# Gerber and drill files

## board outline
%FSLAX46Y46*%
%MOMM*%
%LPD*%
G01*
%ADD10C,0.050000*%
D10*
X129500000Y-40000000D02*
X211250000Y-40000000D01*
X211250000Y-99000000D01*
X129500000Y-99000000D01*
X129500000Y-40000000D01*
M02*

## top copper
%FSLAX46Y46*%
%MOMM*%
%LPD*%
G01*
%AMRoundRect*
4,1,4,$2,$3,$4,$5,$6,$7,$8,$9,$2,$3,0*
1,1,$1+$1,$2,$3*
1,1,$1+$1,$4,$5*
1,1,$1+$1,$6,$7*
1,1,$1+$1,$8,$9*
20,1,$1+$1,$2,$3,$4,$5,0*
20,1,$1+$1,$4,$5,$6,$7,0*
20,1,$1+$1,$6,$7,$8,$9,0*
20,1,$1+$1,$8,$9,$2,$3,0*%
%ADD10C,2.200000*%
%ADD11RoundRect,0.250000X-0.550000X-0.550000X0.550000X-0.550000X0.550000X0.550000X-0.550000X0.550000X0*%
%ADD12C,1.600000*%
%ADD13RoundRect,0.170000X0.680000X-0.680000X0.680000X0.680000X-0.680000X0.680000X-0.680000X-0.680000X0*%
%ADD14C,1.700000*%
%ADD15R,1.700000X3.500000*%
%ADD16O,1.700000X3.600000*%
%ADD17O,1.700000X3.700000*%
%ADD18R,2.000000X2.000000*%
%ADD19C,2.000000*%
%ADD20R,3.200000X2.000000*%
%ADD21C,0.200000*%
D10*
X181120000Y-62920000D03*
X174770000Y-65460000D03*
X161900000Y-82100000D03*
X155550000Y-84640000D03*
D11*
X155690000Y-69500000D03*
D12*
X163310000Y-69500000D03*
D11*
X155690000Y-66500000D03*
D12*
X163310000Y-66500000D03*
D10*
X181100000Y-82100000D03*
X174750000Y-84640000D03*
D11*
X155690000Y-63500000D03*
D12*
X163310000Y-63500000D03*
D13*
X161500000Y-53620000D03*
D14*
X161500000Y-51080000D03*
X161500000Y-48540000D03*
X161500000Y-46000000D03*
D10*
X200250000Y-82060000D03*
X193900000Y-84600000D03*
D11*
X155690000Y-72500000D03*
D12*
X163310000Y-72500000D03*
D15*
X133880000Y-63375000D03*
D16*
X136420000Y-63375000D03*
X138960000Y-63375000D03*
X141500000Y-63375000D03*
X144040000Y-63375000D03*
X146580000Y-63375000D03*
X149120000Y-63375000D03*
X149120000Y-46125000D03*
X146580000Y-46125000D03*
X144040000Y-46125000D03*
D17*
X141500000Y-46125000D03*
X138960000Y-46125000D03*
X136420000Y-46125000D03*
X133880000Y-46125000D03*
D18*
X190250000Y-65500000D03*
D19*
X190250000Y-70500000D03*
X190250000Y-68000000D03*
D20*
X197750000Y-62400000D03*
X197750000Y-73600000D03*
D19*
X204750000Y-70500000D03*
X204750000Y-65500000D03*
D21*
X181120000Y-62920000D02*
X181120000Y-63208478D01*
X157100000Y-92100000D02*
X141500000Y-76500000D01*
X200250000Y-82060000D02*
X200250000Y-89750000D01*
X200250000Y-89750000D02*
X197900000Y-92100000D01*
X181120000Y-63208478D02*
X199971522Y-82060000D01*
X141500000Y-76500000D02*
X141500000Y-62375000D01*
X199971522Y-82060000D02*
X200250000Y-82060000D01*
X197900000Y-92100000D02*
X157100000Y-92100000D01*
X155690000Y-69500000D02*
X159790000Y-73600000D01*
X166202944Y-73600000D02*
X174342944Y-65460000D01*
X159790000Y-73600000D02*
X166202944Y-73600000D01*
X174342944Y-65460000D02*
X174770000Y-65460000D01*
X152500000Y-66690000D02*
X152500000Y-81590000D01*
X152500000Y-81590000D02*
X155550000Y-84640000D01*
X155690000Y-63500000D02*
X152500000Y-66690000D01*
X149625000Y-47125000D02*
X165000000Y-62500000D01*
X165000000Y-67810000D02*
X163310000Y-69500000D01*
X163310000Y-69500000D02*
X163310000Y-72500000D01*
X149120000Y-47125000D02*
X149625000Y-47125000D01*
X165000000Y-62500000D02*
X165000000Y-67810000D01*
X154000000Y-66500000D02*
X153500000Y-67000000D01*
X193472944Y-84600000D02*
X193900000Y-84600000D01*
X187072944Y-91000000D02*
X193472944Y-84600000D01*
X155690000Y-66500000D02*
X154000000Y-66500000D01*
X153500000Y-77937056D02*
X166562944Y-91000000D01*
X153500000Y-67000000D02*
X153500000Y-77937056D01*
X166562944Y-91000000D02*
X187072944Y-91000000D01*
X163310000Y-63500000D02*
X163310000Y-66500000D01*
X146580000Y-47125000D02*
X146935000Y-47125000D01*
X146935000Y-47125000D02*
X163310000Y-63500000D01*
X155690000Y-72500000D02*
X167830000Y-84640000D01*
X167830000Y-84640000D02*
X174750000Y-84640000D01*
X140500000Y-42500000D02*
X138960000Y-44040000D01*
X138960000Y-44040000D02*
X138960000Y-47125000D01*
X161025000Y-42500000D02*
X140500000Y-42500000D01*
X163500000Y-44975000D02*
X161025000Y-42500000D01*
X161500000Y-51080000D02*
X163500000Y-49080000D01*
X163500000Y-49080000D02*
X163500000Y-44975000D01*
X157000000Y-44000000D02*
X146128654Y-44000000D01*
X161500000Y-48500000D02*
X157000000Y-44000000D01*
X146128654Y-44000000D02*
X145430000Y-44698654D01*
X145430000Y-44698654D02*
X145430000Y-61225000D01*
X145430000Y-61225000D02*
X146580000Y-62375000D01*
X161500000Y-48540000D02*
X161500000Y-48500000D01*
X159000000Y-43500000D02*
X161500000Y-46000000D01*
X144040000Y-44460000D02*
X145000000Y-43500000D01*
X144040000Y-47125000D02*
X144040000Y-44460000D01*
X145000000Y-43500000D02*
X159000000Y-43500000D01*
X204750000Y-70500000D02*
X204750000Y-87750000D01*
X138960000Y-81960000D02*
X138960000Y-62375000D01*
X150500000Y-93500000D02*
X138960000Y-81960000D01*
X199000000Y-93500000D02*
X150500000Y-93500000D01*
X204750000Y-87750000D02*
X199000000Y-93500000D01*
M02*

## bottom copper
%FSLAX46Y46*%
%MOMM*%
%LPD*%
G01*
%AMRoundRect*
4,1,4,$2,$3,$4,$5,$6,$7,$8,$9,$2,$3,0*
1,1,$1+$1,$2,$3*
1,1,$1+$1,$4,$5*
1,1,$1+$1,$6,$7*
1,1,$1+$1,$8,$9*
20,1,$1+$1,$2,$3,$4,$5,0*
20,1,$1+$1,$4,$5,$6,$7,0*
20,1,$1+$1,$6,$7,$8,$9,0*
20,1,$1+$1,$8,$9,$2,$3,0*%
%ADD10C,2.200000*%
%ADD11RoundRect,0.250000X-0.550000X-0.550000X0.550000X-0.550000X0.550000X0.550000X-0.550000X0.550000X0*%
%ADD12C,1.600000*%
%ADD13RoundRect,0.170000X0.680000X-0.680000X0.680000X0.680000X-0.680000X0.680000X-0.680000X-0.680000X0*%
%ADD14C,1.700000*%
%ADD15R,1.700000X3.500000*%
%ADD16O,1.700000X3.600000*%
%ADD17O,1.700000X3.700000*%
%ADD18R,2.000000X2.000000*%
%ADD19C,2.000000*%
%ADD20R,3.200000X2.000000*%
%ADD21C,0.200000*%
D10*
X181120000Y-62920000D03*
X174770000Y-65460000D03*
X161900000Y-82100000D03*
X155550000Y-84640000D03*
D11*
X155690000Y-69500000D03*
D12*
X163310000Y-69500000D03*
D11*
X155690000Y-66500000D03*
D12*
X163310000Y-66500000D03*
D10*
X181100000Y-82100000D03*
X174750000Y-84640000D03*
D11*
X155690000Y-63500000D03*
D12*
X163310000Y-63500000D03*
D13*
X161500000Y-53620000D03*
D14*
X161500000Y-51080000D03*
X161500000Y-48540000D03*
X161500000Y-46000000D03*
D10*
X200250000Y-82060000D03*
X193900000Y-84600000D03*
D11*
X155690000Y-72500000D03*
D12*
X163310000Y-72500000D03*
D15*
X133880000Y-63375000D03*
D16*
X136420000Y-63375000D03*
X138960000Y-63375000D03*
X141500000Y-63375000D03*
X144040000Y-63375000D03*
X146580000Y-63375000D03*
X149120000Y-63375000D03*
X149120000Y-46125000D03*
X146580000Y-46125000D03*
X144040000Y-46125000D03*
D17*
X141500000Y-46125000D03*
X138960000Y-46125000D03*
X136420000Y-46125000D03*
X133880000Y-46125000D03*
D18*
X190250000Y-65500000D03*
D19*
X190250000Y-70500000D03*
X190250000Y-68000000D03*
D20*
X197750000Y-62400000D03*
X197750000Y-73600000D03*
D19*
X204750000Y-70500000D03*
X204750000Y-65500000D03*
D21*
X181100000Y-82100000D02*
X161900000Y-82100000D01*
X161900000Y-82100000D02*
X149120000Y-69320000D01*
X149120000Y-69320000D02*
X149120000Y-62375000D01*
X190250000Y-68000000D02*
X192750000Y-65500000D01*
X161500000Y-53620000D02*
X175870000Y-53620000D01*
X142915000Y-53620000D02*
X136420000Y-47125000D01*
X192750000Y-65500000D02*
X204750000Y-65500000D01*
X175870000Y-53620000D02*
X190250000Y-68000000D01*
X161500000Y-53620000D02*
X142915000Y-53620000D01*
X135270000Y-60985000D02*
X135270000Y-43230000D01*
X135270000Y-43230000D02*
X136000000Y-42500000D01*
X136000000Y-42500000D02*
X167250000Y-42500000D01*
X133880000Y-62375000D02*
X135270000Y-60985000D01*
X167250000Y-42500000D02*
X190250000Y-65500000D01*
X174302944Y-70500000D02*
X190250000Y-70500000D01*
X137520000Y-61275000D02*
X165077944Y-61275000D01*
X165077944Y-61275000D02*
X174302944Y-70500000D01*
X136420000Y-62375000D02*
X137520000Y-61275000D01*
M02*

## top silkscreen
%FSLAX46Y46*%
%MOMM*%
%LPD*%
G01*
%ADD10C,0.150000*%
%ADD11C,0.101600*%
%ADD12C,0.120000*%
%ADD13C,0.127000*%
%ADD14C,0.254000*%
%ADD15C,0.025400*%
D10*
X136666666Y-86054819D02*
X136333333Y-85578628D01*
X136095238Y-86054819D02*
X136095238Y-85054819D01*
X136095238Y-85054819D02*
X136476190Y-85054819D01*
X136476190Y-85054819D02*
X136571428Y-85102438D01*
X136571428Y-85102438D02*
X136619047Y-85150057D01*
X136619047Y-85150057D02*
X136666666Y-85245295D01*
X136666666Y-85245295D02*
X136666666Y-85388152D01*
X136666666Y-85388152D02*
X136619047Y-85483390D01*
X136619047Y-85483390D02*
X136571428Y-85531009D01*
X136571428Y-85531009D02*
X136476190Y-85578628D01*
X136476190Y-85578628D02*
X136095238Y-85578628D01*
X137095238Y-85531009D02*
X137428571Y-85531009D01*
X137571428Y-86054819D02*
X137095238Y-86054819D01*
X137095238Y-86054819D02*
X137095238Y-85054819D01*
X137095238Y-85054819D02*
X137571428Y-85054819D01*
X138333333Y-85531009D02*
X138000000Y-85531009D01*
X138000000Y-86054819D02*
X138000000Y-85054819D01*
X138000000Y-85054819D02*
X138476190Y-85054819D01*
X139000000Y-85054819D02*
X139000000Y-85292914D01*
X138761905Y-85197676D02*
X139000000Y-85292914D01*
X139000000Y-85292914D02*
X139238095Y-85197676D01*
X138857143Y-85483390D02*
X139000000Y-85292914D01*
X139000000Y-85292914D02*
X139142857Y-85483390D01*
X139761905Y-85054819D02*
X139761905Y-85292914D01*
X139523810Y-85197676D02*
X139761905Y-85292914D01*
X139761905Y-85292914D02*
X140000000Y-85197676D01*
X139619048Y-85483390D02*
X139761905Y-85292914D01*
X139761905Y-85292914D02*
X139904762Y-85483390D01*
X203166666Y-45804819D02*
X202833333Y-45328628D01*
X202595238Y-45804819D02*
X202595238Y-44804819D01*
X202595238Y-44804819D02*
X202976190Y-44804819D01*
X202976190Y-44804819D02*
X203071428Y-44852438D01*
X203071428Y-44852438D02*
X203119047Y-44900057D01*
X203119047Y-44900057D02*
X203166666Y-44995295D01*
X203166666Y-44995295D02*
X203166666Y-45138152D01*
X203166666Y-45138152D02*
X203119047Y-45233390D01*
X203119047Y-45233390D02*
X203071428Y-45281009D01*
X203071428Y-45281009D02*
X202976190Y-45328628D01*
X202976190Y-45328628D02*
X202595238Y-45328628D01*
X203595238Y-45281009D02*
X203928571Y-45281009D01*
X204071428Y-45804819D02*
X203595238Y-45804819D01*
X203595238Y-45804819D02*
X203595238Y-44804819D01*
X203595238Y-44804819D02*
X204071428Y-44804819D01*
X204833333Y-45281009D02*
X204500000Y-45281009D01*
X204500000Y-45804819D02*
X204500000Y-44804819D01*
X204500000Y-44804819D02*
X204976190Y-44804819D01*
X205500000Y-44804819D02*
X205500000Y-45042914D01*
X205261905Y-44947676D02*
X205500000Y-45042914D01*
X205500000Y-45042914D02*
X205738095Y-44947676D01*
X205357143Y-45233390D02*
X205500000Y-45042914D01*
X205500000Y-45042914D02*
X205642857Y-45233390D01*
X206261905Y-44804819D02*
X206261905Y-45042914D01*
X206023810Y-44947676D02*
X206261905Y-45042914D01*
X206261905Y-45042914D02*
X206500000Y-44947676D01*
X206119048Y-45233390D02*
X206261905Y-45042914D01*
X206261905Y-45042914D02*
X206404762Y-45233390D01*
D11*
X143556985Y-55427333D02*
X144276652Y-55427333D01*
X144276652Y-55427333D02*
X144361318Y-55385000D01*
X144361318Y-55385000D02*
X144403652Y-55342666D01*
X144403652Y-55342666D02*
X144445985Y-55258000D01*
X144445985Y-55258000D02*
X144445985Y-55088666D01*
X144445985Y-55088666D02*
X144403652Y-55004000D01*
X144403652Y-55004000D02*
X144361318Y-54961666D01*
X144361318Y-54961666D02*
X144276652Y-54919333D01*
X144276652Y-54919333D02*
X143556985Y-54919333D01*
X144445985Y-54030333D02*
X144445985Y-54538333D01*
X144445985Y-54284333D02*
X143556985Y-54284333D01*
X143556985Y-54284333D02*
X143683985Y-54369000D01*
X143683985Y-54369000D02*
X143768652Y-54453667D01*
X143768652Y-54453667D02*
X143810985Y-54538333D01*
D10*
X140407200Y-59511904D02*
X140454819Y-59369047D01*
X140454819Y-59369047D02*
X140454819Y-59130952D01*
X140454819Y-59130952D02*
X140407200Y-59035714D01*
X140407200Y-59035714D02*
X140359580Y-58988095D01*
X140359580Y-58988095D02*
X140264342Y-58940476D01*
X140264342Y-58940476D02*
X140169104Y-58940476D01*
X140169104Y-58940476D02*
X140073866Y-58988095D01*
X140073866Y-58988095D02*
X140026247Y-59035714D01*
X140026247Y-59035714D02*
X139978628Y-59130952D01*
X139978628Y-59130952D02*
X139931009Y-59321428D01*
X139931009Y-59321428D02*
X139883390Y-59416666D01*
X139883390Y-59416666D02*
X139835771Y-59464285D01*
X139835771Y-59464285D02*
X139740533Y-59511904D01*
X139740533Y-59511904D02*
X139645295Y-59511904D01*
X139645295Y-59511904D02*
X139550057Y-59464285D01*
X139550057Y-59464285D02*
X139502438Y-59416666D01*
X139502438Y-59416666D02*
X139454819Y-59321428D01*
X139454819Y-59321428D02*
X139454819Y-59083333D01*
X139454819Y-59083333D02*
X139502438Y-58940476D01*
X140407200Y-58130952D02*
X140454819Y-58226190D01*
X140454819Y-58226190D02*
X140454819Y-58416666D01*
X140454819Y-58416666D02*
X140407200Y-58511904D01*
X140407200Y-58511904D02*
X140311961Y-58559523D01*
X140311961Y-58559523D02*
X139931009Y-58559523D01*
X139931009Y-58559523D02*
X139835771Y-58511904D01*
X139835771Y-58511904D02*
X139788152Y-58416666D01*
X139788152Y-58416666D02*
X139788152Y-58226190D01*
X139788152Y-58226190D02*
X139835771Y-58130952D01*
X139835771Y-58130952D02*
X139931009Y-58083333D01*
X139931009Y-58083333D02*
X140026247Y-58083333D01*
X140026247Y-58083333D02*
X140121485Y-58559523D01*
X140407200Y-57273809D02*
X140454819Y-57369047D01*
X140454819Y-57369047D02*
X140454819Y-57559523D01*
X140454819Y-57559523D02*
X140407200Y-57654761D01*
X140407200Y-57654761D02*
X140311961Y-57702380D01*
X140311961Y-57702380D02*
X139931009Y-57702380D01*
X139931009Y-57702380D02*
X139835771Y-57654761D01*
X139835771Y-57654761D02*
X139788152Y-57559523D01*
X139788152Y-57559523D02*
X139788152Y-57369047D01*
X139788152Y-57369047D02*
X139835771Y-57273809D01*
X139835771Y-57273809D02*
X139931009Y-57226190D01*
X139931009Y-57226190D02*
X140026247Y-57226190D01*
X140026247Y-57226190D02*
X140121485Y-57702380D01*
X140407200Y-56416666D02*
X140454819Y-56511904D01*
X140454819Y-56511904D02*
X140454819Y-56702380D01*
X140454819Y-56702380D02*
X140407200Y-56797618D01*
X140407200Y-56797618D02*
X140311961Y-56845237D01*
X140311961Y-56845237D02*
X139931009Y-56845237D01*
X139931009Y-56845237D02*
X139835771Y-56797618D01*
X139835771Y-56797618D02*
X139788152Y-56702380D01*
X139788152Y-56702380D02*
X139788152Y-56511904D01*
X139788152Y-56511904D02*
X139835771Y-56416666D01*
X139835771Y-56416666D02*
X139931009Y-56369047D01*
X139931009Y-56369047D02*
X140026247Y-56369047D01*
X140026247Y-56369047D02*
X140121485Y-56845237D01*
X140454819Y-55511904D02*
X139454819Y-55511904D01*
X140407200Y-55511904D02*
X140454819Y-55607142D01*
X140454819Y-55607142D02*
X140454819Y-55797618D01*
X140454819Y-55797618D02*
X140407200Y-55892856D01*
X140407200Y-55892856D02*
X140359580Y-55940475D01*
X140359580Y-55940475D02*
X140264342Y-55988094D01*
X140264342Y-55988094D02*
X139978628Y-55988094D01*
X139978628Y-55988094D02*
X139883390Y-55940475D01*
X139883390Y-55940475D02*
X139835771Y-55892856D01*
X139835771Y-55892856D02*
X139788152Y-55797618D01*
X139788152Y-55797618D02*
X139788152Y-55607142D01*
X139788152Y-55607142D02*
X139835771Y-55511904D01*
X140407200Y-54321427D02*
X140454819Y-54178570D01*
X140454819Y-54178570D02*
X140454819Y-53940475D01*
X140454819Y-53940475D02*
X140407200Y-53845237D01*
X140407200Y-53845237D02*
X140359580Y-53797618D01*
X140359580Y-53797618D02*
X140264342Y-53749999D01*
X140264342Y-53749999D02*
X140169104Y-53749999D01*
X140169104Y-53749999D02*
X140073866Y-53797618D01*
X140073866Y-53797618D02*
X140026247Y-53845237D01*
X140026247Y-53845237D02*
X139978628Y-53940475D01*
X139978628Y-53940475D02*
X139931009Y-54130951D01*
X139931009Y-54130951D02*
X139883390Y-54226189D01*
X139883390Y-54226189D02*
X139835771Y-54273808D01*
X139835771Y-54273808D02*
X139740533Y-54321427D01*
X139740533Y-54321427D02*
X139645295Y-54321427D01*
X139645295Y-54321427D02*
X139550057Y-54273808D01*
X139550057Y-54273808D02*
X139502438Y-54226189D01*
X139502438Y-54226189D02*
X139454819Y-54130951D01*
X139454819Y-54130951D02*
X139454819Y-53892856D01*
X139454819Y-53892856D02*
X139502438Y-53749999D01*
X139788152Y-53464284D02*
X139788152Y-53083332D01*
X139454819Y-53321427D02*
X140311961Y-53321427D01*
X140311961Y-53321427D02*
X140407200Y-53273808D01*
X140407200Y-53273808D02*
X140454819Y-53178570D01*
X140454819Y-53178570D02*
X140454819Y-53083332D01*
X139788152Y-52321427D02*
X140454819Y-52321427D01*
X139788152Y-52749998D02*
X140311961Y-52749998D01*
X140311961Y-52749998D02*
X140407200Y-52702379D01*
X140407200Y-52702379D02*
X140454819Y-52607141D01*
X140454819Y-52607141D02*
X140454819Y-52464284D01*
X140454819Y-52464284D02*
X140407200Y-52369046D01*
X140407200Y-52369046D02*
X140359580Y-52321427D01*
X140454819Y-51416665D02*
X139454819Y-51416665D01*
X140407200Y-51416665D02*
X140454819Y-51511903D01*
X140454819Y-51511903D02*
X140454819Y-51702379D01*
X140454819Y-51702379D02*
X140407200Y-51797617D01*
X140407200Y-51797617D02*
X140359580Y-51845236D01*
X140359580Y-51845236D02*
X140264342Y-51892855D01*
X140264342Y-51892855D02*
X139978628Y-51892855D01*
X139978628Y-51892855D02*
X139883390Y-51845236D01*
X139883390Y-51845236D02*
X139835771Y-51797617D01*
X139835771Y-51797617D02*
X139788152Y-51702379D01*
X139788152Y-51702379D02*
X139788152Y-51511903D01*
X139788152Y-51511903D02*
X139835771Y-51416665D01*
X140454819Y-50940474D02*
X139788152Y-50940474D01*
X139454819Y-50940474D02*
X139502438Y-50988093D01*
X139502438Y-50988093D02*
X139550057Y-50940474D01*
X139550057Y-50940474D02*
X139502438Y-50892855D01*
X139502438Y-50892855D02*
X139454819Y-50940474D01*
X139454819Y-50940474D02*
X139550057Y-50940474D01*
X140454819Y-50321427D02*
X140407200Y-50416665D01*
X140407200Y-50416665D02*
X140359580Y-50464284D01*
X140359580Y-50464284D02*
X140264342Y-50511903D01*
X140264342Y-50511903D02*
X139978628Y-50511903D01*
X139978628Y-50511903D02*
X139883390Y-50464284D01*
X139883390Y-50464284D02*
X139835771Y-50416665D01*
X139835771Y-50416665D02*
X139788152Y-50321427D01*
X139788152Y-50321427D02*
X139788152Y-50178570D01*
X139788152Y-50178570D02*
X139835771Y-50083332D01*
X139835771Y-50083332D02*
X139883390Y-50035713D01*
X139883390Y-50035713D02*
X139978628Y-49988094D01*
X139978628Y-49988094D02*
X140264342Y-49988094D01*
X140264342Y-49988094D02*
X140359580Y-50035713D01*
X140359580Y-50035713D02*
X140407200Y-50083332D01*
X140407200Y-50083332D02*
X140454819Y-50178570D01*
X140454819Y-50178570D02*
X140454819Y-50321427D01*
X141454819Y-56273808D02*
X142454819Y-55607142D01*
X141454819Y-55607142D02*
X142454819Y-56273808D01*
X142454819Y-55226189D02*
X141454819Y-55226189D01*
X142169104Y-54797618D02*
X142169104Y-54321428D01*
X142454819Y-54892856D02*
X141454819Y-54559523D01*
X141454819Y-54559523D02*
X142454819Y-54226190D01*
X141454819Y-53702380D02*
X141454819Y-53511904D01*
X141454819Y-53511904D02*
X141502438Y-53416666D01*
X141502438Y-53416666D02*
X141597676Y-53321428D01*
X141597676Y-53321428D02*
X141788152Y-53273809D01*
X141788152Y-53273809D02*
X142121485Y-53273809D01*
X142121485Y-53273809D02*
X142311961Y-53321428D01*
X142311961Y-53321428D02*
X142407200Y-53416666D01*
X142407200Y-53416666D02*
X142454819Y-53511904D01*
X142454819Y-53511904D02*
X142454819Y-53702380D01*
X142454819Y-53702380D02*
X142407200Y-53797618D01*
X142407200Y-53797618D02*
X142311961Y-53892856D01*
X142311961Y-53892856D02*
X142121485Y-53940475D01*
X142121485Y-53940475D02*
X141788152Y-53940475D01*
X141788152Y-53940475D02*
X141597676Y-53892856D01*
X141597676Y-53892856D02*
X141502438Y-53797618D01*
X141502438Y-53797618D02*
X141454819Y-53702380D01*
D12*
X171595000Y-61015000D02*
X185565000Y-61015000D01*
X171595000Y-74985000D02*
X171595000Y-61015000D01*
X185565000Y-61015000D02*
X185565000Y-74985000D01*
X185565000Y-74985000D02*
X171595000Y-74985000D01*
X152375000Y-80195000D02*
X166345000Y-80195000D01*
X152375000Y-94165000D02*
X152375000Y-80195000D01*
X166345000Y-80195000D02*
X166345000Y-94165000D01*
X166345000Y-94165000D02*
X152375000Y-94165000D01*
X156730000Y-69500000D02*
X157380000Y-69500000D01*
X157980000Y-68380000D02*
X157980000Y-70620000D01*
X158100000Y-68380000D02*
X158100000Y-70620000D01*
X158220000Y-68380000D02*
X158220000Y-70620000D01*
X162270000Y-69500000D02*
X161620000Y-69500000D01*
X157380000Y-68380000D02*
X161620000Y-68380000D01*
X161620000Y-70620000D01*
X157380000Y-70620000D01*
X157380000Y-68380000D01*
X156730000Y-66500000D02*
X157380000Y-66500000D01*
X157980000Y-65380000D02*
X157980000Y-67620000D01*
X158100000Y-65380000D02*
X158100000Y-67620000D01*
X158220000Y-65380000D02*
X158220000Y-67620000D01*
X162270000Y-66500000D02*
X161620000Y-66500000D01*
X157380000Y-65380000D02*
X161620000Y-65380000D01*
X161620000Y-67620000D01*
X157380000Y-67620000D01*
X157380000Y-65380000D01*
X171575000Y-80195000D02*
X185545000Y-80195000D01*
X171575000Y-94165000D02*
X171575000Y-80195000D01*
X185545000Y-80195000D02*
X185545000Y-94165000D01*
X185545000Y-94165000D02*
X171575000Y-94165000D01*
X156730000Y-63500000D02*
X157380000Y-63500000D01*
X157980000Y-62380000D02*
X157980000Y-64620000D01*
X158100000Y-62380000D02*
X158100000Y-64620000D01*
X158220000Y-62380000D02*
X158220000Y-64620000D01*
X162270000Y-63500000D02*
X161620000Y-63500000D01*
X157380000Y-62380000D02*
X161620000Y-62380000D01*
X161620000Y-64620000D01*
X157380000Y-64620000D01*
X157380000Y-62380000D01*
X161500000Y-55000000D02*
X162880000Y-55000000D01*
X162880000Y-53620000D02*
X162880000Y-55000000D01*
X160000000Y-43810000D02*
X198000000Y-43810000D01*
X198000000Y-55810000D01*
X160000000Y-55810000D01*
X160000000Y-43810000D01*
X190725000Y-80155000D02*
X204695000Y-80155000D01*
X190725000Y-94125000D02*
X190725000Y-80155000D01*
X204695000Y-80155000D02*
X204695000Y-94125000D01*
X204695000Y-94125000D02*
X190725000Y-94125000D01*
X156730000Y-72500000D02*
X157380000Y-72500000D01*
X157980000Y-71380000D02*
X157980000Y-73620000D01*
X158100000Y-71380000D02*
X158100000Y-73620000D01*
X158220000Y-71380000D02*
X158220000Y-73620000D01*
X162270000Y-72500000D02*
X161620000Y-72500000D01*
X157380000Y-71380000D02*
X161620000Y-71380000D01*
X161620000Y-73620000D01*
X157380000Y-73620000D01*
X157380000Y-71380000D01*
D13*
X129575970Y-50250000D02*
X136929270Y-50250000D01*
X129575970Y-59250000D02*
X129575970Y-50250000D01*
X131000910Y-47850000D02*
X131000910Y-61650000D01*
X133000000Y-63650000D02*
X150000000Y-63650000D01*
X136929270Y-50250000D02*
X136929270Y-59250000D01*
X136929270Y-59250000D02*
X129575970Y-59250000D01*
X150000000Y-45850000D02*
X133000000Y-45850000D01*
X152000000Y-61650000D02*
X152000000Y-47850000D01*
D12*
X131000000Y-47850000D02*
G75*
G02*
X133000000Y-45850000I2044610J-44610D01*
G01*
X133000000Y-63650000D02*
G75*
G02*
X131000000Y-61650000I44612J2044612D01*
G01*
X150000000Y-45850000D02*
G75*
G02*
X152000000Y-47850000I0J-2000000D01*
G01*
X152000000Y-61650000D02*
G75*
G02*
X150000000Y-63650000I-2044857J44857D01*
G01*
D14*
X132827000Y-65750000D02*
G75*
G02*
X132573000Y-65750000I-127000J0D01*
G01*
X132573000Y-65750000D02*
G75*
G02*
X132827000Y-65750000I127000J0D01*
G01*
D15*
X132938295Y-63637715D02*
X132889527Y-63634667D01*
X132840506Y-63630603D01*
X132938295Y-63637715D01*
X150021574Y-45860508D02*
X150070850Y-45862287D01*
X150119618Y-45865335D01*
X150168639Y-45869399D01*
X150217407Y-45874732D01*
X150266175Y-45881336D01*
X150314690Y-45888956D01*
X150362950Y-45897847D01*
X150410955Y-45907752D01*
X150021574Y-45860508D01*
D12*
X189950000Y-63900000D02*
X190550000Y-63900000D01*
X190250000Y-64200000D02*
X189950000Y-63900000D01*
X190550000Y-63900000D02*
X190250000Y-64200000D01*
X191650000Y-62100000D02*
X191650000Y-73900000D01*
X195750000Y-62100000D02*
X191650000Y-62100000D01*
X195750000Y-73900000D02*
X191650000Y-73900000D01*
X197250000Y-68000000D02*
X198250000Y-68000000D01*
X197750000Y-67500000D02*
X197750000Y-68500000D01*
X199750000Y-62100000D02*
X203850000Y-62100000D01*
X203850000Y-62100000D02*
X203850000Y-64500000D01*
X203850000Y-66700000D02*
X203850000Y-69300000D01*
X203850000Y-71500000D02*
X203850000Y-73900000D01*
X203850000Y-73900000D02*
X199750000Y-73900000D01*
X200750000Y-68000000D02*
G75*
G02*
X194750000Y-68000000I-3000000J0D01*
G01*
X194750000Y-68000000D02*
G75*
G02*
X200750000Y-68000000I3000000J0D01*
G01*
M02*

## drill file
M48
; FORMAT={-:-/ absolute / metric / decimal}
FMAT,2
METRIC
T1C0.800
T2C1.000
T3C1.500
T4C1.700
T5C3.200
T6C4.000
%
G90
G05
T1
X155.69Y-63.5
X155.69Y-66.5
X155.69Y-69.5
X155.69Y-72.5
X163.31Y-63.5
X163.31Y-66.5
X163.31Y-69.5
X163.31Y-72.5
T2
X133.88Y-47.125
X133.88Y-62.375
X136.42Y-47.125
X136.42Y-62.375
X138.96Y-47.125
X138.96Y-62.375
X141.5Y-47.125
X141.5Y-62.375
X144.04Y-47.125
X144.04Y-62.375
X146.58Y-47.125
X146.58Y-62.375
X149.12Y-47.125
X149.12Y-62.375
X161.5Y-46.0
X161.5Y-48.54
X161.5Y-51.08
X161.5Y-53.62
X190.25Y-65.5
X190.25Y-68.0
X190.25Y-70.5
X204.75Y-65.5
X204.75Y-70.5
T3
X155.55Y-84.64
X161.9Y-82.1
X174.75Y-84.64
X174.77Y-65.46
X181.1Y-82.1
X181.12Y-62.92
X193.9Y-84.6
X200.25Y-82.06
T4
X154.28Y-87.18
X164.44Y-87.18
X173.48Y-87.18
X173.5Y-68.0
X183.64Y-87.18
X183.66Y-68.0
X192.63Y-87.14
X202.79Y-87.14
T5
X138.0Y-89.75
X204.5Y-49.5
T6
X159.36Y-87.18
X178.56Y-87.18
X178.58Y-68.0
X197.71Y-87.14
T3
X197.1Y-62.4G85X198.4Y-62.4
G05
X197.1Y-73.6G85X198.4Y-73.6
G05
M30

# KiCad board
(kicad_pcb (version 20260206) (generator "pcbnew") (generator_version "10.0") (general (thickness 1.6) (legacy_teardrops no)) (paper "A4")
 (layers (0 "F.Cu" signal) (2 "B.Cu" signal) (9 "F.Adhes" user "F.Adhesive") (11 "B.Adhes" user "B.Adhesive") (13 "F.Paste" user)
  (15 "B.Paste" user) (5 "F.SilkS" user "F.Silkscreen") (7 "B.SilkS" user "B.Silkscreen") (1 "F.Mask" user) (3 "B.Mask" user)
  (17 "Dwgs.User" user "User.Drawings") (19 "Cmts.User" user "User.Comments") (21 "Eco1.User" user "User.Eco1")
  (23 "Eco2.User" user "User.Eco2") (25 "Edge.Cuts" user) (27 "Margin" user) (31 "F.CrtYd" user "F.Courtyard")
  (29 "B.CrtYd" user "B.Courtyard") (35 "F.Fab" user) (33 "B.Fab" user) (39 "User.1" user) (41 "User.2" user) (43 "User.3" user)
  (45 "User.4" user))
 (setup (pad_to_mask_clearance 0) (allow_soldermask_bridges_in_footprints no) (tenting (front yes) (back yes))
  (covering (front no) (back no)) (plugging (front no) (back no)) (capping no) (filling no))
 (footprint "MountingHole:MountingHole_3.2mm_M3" (layer "F.Cu") (at 138 89.75)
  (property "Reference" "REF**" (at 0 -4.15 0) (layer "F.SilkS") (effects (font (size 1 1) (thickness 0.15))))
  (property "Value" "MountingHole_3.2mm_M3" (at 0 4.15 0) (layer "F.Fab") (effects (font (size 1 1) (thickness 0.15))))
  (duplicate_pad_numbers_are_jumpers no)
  (pad "" np_thru_hole circle (at 0 0) (size 3.2 3.2) (drill 3.2) (layers "*.Cu" "*.Mask")))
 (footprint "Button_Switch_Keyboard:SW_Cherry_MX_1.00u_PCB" (layer "F.Cu") (at 181.12 62.92)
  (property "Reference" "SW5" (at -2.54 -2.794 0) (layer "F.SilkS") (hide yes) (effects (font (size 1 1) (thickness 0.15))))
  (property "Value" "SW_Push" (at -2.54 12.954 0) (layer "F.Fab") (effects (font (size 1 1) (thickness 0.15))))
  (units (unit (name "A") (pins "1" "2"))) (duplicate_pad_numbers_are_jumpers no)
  (fp_line (start -9.525 -1.905) (end 4.445 -1.905) (stroke (width 0.12) (type solid)) (layer "F.SilkS"))
  (fp_line (start -9.525 12.065) (end -9.525 -1.905) (stroke (width 0.12) (type solid)) (layer "F.SilkS"))
  (fp_line (start 4.445 -1.905) (end 4.445 12.065) (stroke (width 0.12) (type solid)) (layer "F.SilkS"))
  (fp_line (start 4.445 12.065) (end -9.525 12.065) (stroke (width 0.12) (type solid)) (layer "F.SilkS"))
  (pad "" np_thru_hole circle (at -7.62 5.08) (size 1.7 1.7) (drill 1.7) (layers "*.Cu" "*.Mask"))
  (pad "" np_thru_hole circle (at -2.54 5.08) (size 4 4) (drill 4) (layers "*.Cu" "*.Mask"))
  (pad "" np_thru_hole circle (at 2.54 5.08) (size 1.7 1.7) (drill 1.7) (layers "*.Cu" "*.Mask"))
  (pad "1" thru_hole circle (at 0 0) (size 2.2 2.2) (drill 1.5) (layers "*.Cu" "*.Mask") (remove_unused_layers no)
   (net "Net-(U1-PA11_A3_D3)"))
  (pad "2" thru_hole circle (at -6.35 2.54) (size 2.2 2.2) (drill 1.5) (layers "*.Cu" "*.Mask") (remove_unused_layers no) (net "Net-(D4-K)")))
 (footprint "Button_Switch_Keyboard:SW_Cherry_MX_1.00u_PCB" (layer "F.Cu") (at 161.9 82.1)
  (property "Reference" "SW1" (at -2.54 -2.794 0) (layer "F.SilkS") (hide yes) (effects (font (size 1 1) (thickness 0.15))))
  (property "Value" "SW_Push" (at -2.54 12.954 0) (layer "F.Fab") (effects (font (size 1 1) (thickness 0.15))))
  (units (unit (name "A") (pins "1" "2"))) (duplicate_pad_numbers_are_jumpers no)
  (fp_line (start -9.525 -1.905) (end 4.445 -1.905) (stroke (width 0.12) (type solid)) (layer "F.SilkS"))
  (fp_line (start -9.525 12.065) (end -9.525 -1.905) (stroke (width 0.12) (type solid)) (layer "F.SilkS"))
  (fp_line (start 4.445 -1.905) (end 4.445 12.065) (stroke (width 0.12) (type solid)) (layer "F.SilkS"))
  (fp_line (start 4.445 12.065) (end -9.525 12.065) (stroke (width 0.12) (type solid)) (layer "F.SilkS"))
  (pad "" np_thru_hole circle (at -7.62 5.08) (size 1.7 1.7) (drill 1.7) (layers "*.Cu" "*.Mask"))
  (pad "" np_thru_hole circle (at -2.54 5.08) (size 4 4) (drill 4) (layers "*.Cu" "*.Mask"))
  (pad "" np_thru_hole circle (at 2.54 5.08) (size 1.7 1.7) (drill 1.7) (layers "*.Cu" "*.Mask"))
  (pad "1" thru_hole circle (at 0 0) (size 2.2 2.2) (drill 1.5) (layers "*.Cu" "*.Mask") (remove_unused_layers no)
   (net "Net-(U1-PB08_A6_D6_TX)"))
  (pad "2" thru_hole circle (at -6.35 2.54) (size 2.2 2.2) (drill 1.5) (layers "*.Cu" "*.Mask") (remove_unused_layers no) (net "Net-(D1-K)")))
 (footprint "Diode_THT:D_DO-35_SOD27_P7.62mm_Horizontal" (layer "F.Cu") (at 155.69 69.5)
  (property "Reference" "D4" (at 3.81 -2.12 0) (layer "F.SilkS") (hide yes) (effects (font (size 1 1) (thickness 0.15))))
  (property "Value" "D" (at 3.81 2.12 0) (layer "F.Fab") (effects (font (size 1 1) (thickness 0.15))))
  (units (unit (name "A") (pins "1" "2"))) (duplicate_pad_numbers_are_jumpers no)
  (fp_line (start 1.04 0) (end 1.69 0) (stroke (width 0.12) (type solid)) (layer "F.SilkS"))
  (fp_line (start 2.29 -1.12) (end 2.29 1.12) (stroke (width 0.12) (type solid)) (layer "F.SilkS"))
  (fp_line (start 2.41 -1.12) (end 2.41 1.12) (stroke (width 0.12) (type solid)) (layer "F.SilkS"))
  (fp_line (start 2.53 -1.12) (end 2.53 1.12) (stroke (width 0.12) (type solid)) (layer "F.SilkS"))
  (fp_line (start 6.58 0) (end 5.93 0) (stroke (width 0.12) (type solid)) (layer "F.SilkS"))
  (fp_rect (start 1.69 -1.12) (end 5.93 1.12) (stroke (width 0.12) (type solid)) (fill no) (layer "F.SilkS"))
  (pad "1" thru_hole roundrect (at 0 0) (size 1.6 1.6) (drill 0.8) (layers "*.Cu" "*.Mask") (remove_unused_layers no)
   (roundrect_rratio 0.15625) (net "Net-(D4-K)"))
  (pad "2" thru_hole circle (at 7.62 0) (size 1.6 1.6) (drill 0.8) (layers "*.Cu" "*.Mask") (remove_unused_layers no) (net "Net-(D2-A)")))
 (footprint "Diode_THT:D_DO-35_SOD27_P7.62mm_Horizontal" (layer "F.Cu") (at 155.69 66.5)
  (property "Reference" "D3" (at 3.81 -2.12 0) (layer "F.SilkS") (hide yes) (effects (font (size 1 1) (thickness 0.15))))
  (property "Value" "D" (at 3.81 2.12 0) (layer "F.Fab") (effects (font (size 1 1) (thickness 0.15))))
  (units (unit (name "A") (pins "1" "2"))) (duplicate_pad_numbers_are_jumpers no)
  (fp_line (start 1.04 0) (end 1.69 0) (stroke (width 0.12) (type solid)) (layer "F.SilkS"))
  (fp_line (start 2.29 -1.12) (end 2.29 1.12) (stroke (width 0.12) (type solid)) (layer "F.SilkS"))
  (fp_line (start 2.41 -1.12) (end 2.41 1.12) (stroke (width 0.12) (type solid)) (layer "F.SilkS"))
  (fp_line (start 2.53 -1.12) (end 2.53 1.12) (stroke (width 0.12) (type solid)) (layer "F.SilkS"))
  (fp_line (start 6.58 0) (end 5.93 0) (stroke (width 0.12) (type solid)) (layer "F.SilkS"))
  (fp_rect (start 1.69 -1.12) (end 5.93 1.12) (stroke (width 0.12) (type solid)) (fill no) (layer "F.SilkS"))
  (pad "1" thru_hole roundrect (at 0 0) (size 1.6 1.6) (drill 0.8) (layers "*.Cu" "*.Mask") (remove_unused_layers no)
   (roundrect_rratio 0.15625) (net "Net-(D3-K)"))
  (pad "2" thru_hole circle (at 7.62 0) (size 1.6 1.6) (drill 0.8) (layers "*.Cu" "*.Mask") (remove_unused_layers no) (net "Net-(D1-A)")))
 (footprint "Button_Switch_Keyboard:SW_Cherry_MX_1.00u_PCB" (layer "F.Cu") (at 181.1 82.1)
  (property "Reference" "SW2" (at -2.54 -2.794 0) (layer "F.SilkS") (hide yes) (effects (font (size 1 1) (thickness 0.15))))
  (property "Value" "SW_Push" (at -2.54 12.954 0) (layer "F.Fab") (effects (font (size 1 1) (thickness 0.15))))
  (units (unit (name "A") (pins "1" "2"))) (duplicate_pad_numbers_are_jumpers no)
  (fp_line (start -9.525 -1.905) (end 4.445 -1.905) (stroke (width 0.12) (type solid)) (layer "F.SilkS"))
  (fp_line (start -9.525 12.065) (end -9.525 -1.905) (stroke (width 0.12) (type solid)) (layer "F.SilkS"))
  (fp_line (start 4.445 -1.905) (end 4.445 12.065) (stroke (width 0.12) (type solid)) (layer "F.SilkS"))
  (fp_line (start 4.445 12.065) (end -9.525 12.065) (stroke (width 0.12) (type solid)) (layer "F.SilkS"))
  (pad "" np_thru_hole circle (at -7.62 5.08) (size 1.7 1.7) (drill 1.7) (layers "*.Cu" "*.Mask"))
  (pad "" np_thru_hole circle (at -2.54 5.08) (size 4 4) (drill 4) (layers "*.Cu" "*.Mask"))
  (pad "" np_thru_hole circle (at 2.54 5.08) (size 1.7 1.7) (drill 1.7) (layers "*.Cu" "*.Mask"))
  (pad "1" thru_hole circle (at 0 0) (size 2.2 2.2) (drill 1.5) (layers "*.Cu" "*.Mask") (remove_unused_layers no)
   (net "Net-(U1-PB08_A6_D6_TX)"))
  (pad "2" thru_hole circle (at -6.35 2.54) (size 2.2 2.2) (drill 1.5) (layers "*.Cu" "*.Mask") (remove_unused_layers no) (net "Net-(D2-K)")))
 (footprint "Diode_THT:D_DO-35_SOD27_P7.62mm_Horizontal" (layer "F.Cu") (at 155.69 63.5)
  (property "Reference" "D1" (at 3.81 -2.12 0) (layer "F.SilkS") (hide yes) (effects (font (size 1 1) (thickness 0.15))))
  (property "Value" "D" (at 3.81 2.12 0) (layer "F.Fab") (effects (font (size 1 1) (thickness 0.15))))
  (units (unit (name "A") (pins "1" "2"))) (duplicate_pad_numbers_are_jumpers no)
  (fp_line (start 1.04 0) (end 1.69 0) (stroke (width 0.12) (type solid)) (layer "F.SilkS"))
  (fp_line (start 2.29 -1.12) (end 2.29 1.12) (stroke (width 0.12) (type solid)) (layer "F.SilkS"))
  (fp_line (start 2.41 -1.12) (end 2.41 1.12) (stroke (width 0.12) (type solid)) (layer "F.SilkS"))
  (fp_line (start 2.53 -1.12) (end 2.53 1.12) (stroke (width 0.12) (type solid)) (layer "F.SilkS"))
  (fp_line (start 6.58 0) (end 5.93 0) (stroke (width 0.12) (type solid)) (layer "F.SilkS"))
  (fp_rect (start 1.69 -1.12) (end 5.93 1.12) (stroke (width 0.12) (type solid)) (fill no) (layer "F.SilkS"))
  (pad "1" thru_hole roundrect (at 0 0) (size 1.6 1.6) (drill 0.8) (layers "*.Cu" "*.Mask") (remove_unused_layers no)
   (roundrect_rratio 0.15625) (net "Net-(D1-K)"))
  (pad "2" thru_hole circle (at 7.62 0) (size 1.6 1.6) (drill 0.8) (layers "*.Cu" "*.Mask") (remove_unused_layers no) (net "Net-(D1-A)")))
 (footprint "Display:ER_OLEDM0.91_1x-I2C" (layer "F.Cu") (at 161.5 53.62 90)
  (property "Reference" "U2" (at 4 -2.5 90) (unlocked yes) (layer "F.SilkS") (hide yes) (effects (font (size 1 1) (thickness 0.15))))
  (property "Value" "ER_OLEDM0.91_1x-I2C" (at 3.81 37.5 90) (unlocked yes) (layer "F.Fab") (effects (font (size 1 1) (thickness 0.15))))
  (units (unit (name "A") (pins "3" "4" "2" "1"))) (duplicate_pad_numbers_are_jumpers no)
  (fp_line (start -1.38 0) (end -1.38 1.38) (stroke (width 0.12) (type solid)) (layer "F.SilkS"))
  (fp_line (start 0 1.38) (end -1.38 1.38) (stroke (width 0.12) (type solid)) (layer "F.SilkS"))
  (fp_rect (start -2.19 -1.5) (end 9.81 36.5) (stroke (width 0.12) (type solid)) (fill no) (layer "F.SilkS"))
  (pad "1" thru_hole roundrect (at 0 0 90) (size 1.7 1.7) (drill 1) (layers "*.Cu" "*.Mask") (remove_unused_layers no)
   (roundrect_rratio 0.1) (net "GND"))
  (pad "2" thru_hole circle (at 2.54 0 90) (size 1.7 1.7) (drill 1) (layers "*.Cu" "*.Mask") (remove_unused_layers no) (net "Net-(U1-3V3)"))
  (pad "3" thru_hole circle (at 5.08 0 90) (size 1.7 1.7) (drill 1) (layers "*.Cu" "*.Mask") (remove_unused_layers no)
   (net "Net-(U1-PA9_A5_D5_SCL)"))
  (pad "4" thru_hole circle (at 7.62 0 90) (size 1.7 1.7) (drill 1) (layers "*.Cu" "*.Mask") (remove_unused_layers no)
   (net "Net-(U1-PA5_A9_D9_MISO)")))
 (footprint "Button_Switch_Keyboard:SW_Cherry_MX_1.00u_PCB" (layer "F.Cu") (at 200.25 82.06)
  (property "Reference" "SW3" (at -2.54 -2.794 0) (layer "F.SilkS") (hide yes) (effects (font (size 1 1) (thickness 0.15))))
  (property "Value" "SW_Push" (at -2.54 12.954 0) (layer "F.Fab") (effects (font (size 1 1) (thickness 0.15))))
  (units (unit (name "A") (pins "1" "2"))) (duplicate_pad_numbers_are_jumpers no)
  (fp_line (start -9.525 -1.905) (end 4.445 -1.905) (stroke (width 0.12) (type solid)) (layer "F.SilkS"))
  (fp_line (start -9.525 12.065) (end -9.525 -1.905) (stroke (width 0.12) (type solid)) (layer "F.SilkS"))
  (fp_line (start 4.445 -1.905) (end 4.445 12.065) (stroke (width 0.12) (type solid)) (layer "F.SilkS"))
  (fp_line (start 4.445 12.065) (end -9.525 12.065) (stroke (width 0.12) (type solid)) (layer "F.SilkS"))
  (pad "" np_thru_hole circle (at -7.62 5.08) (size 1.7 1.7) (drill 1.7) (layers "*.Cu" "*.Mask"))
  (pad "" np_thru_hole circle (at -2.54 5.08) (size 4 4) (drill 4) (layers "*.Cu" "*.Mask"))
  (pad "" np_thru_hole circle (at 2.54 5.08) (size 1.7 1.7) (drill 1.7) (layers "*.Cu" "*.Mask"))
  (pad "1" thru_hole circle (at 0 0) (size 2.2 2.2) (drill 1.5) (layers "*.Cu" "*.Mask") (remove_unused_layers no)
   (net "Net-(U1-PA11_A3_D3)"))
  (pad "2" thru_hole circle (at -6.35 2.54) (size 2.2 2.2) (drill 1.5) (layers "*.Cu" "*.Mask") (remove_unused_layers no) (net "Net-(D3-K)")))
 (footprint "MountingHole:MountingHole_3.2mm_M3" (layer "F.Cu") (at 204.5 49.5)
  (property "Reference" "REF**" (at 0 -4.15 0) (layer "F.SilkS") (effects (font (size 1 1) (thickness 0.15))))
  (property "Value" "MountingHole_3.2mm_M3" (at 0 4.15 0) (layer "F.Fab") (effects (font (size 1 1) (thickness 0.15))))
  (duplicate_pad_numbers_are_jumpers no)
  (pad "" np_thru_hole circle (at 0 0) (size 3.2 3.2) (drill 3.2) (layers "*.Cu" "*.Mask")))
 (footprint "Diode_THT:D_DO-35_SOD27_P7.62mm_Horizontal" (layer "F.Cu") (at 155.69 72.5)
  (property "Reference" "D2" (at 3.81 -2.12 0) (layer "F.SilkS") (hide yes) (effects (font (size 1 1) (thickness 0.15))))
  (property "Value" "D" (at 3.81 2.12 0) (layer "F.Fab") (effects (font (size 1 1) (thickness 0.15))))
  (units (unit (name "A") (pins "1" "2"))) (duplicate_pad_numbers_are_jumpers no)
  (fp_line (start 1.04 0) (end 1.69 0) (stroke (width 0.12) (type solid)) (layer "F.SilkS"))
  (fp_line (start 2.29 -1.12) (end 2.29 1.12) (stroke (width 0.12) (type solid)) (layer "F.SilkS"))
  (fp_line (start 2.41 -1.12) (end 2.41 1.12) (stroke (width 0.12) (type solid)) (layer "F.SilkS"))
  (fp_line (start 2.53 -1.12) (end 2.53 1.12) (stroke (width 0.12) (type solid)) (layer "F.SilkS"))
  (fp_line (start 6.58 0) (end 5.93 0) (stroke (width 0.12) (type solid)) (layer "F.SilkS"))
  (fp_rect (start 1.69 -1.12) (end 5.93 1.12) (stroke (width 0.12) (type solid)) (fill no) (layer "F.SilkS"))
  (pad "1" thru_hole roundrect (at 0 0) (size 1.6 1.6) (drill 0.8) (layers "*.Cu" "*.Mask") (remove_unused_layers no)
   (roundrect_rratio 0.15625) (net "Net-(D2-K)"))
  (pad "2" thru_hole circle (at 7.62 0) (size 1.6 1.6) (drill 0.8) (layers "*.Cu" "*.Mask") (remove_unused_layers no) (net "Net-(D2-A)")))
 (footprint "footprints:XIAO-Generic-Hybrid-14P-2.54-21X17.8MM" (layer "F.Cu") (at 141.5 54.75 90)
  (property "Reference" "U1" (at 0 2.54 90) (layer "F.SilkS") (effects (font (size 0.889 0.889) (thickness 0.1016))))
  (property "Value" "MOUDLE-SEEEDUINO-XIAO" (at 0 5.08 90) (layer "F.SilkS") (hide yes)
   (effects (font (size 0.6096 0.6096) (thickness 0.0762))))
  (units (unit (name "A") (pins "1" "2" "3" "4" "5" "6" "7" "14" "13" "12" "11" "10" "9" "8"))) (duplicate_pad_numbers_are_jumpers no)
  (fp_line (start 4.5 -11.92403) (end 4.5 -4.57073) (stroke (width 0.127) (type solid)) (layer "F.SilkS"))
  (fp_line (start -4.5 -11.92403) (end 4.5 -11.92403) (stroke (width 0.127) (type solid)) (layer "F.SilkS"))
  (fp_line (start 6.9 -10.49909) (end -6.9 -10.49909) (stroke (width 0.127) (type solid)) (layer "F.SilkS"))
  (fp_line (start -8.9 -8.5) (end -8.9 8.5) (stroke (width 0.127) (type solid)) (layer "F.SilkS"))
  (fp_line (start 4.5 -4.57073) (end -4.5 -4.57073) (stroke (width 0.127) (type solid)) (layer "F.SilkS"))
  (fp_line (start -4.5 -4.57073) (end -4.5 -11.92403) (stroke (width 0.127) (type solid)) (layer "F.SilkS"))
  (fp_line (start 8.9 8.5) (end 8.9 -8.5) (stroke (width 0.127) (type solid)) (layer "F.SilkS"))
  (fp_line (start -6.9 10.5) (end 6.9 10.5) (stroke (width 0.127) (type solid)) (layer "F.SilkS"))
  (fp_arc (start 6.9 -10.5) (mid 8.301491 -9.901491) (end 8.9 -8.5) (stroke (width 0.12) (type solid)) (layer "F.SilkS"))
  (fp_arc (start -8.9 -8.5) (mid -8.301491 -9.901491) (end -6.9 -10.5) (stroke (width 0.12) (type solid)) (layer "F.SilkS"))
  (fp_arc (start 8.9 8.5) (mid 8.314214 9.914214) (end 6.9 10.5) (stroke (width 0.12) (type solid)) (layer "F.SilkS"))
  (fp_arc (start -6.9 10.5) (mid -8.301423 9.901423) (end -8.9 8.5) (stroke (width 0.12) (type solid)) (layer "F.SilkS"))
  (fp_circle (center -11 -8.8) (end -11 -9.054) (stroke (width 0) (type solid)) (fill yes) (layer "F.SilkS"))
  (fp_poly
   (pts (xy -8.887715 -8.561705) (xy -8.884667 -8.610473) (xy -8.880603 -8.659494)) (stroke (width 0.0254) (type solid)) (fill no)
   (layer "F.SilkS"))
  (fp_poly
   (pts (xy 8.889492 8.521574) (xy 8.887713 8.57085) (xy 8.884665 8.619618) (xy 8.880601 8.668639) (xy 8.875268 8.717407)
    (xy 8.868664 8.766175) (xy 8.861044 8.81469) (xy 8.852153 8.86295) (xy 8.842248 8.910955))
   (stroke (width 0.0254) (type solid)) (fill no) (layer "F.SilkS"))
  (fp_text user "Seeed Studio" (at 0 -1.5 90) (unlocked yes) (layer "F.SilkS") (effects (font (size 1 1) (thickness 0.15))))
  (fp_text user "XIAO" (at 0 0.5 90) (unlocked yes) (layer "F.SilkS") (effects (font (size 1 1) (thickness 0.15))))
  (pad "1" thru_hole rect (at -7.625 -7.62 90) (size 3.5 1.7) (drill 1 (offset -1 0)) (layers "*.Cu" "*.Mask") (remove_unused_layers no)
   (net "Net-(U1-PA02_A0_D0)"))
  (pad "2" thru_hole oval (at -7.625 -5.08 90) (size 3.6 1.7) (drill 1 (offset -1 0)) (layers "*.Cu" "*.Mask") (remove_unused_layers no)
   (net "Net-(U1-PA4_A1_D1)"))
  (pad "3" thru_hole oval (at -7.625 -2.54 90) (size 3.6 1.7) (drill 1 (offset -1 0)) (layers "*.Cu" "*.Mask") (remove_unused_layers no)
   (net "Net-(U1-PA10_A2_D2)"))
  (pad "4" thru_hole oval (at -7.625 0 90) (size 3.6 1.7) (drill 1 (offset -1 0)) (layers "*.Cu" "*.Mask") (remove_unused_layers no)
   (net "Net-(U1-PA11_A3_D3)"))
  (pad "5" thru_hole oval (at -7.625 2.54 90) (size 3.6 1.7) (drill 1 (offset -1 0)) (layers "*.Cu" "*.Mask") (remove_unused_layers no)
   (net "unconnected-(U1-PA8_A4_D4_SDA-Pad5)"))
  (pad "6" thru_hole oval (at -7.625 5.08 270) (size 3.6 1.7) (drill 1 (offset 1 0)) (layers "*.Cu" "*.Mask") (remove_unused_layers no)
   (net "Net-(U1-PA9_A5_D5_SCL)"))
  (pad "7" thru_hole oval (at -7.625 7.62 90) (size 3.6 1.7) (drill 1 (offset -1 0)) (layers "*.Cu" "*.Mask") (remove_unused_layers no)
   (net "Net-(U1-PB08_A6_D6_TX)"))
  (pad "8" thru_hole oval (at 7.625 7.62 90) (size 3.6 1.7) (drill 1 (offset 1 0)) (layers "*.Cu" "*.Mask") (remove_unused_layers no)
   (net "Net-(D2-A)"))
  (pad "9" thru_hole oval (at 7.625 5.08 90) (size 3.6 1.7) (drill 1 (offset 1 0)) (layers "*.Cu" "*.Mask") (remove_unused_layers no)
   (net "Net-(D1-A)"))
  (pad "10" thru_hole oval (at 7.625 2.54 90) (size 3.6 1.7) (drill 1 (offset 1 0)) (layers "*.Cu" "*.Mask") (remove_unused_layers no)
   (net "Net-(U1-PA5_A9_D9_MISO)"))
  (pad "11" thru_hole oval (at 7.625 0 90) (size 3.7 1.7) (drill 1 (offset 1 0)) (layers "*.Cu" "*.Mask") (remove_unused_layers no)
   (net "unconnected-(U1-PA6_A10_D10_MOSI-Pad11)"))
  (pad "12" thru_hole oval (at 7.625 -2.54 90) (size 3.7 1.7) (drill 1 (offset 1 0)) (layers "*.Cu" "*.Mask") (remove_unused_layers no)
   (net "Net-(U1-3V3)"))
  (pad "13" thru_hole oval (at 7.625 -5.08 90) (size 3.7 1.7) (drill 1 (offset 1 0)) (layers "*.Cu" "*.Mask") (remove_unused_layers no)
   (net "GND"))
  (pad "14" thru_hole oval (at 7.625 -7.62 90) (size 3.7 1.7) (drill 1 (offset 1 0)) (layers "*.Cu" "*.Mask") (remove_unused_layers no)
   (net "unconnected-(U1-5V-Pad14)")))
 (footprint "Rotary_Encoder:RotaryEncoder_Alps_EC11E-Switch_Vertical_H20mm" (layer "F.Cu") (at 190.25 65.5)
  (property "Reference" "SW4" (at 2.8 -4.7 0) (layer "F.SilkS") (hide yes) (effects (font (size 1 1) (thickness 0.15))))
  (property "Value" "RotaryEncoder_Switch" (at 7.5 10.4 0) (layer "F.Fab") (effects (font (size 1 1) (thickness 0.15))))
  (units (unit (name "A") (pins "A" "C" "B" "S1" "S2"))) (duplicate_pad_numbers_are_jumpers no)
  (fp_line (start -0.3 -1.6) (end 0.3 -1.6) (stroke (width 0.12) (type solid)) (layer "F.SilkS"))
  (fp_line (start 0 -1.3) (end -0.3 -1.6) (stroke (width 0.12) (type solid)) (layer "F.SilkS"))
  (fp_line (start 0.3 -1.6) (end 0 -1.3) (stroke (width 0.12) (type solid)) (layer "F.SilkS"))
  (fp_line (start 1.4 -3.4) (end 1.4 8.4) (stroke (width 0.12) (type solid)) (layer "F.SilkS"))
  (fp_line (start 5.5 -3.4) (end 1.4 -3.4) (stroke (width 0.12) (type solid)) (layer "F.SilkS"))
  (fp_line (start 5.5 8.4) (end 1.4 8.4) (stroke (width 0.12) (type solid)) (layer "F.SilkS"))
  (fp_line (start 7 2.5) (end 8 2.5) (stroke (width 0.12) (type solid)) (layer "F.SilkS"))
  (fp_line (start 7.5 2) (end 7.5 3) (stroke (width 0.12) (type solid)) (layer "F.SilkS"))
  (fp_line (start 9.5 -3.4) (end 13.6 -3.4) (stroke (width 0.12) (type solid)) (layer "F.SilkS"))
  (fp_line (start 13.6 -3.4) (end 13.6 -1) (stroke (width 0.12) (type solid)) (layer "F.SilkS"))
  (fp_line (start 13.6 1.2) (end 13.6 3.8) (stroke (width 0.12) (type solid)) (layer "F.SilkS"))
  (fp_line (start 13.6 6) (end 13.6 8.4) (stroke (width 0.12) (type solid)) (layer "F.SilkS"))
  (fp_line (start 13.6 8.4) (end 9.5 8.4) (stroke (width 0.12) (type solid)) (layer "F.SilkS"))
  (fp_circle (center 7.5 2.5) (end 10.5 2.5) (stroke (width 0.12) (type solid)) (fill no) (layer "F.SilkS"))
  (pad "A" thru_hole rect (at 0 0) (size 2 2) (drill 1) (layers "*.Cu" "*.Mask") (remove_unused_layers no) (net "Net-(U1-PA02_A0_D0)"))
  (pad "B" thru_hole circle (at 0 5) (size 2 2) (drill 1) (layers "*.Cu" "*.Mask") (remove_unused_layers no) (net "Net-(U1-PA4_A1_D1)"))
  (pad "C" thru_hole circle (at 0 2.5) (size 2 2) (drill 1) (layers "*.Cu" "*.Mask") (remove_unused_layers no) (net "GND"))
  (pad "MP" thru_hole rect (at 7.5 -3.1) (size 3.2 2) (drill oval 2.8 1.5) (layers "*.Cu" "*.Mask") (remove_unused_layers no))
  (pad "MP" thru_hole rect (at 7.5 8.1) (size 3.2 2) (drill oval 2.8 1.5) (layers "*.Cu" "*.Mask") (remove_unused_layers no))
  (pad "S1" thru_hole circle (at 14.5 5) (size 2 2) (drill 1) (layers "*.Cu" "*.Mask") (remove_unused_layers no) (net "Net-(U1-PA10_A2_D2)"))
  (pad "S2" thru_hole circle (at 14.5 0) (size 2 2) (drill 1) (layers "*.Cu" "*.Mask") (remove_unused_layers no) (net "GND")))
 (gr_rect (start 129.5 40) (end 211.25 99) (stroke (width 0.05) (type default)) (fill no) (layer "Edge.Cuts"))
 (segment (start 181.12 62.92) (end 181.12 63.208478) (width 0.2) (layer "F.Cu") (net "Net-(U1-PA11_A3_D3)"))
 (segment (start 157.1 92.1) (end 141.5 76.5) (width 0.2) (layer "F.Cu") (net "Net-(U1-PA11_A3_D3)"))
 (segment (start 200.25 82.06) (end 200.25 89.75) (width 0.2) (layer "F.Cu") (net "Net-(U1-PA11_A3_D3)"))
 (segment (start 200.25 89.75) (end 197.9 92.1) (width 0.2) (layer "F.Cu") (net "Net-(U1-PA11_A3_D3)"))
 (segment (start 181.12 63.208478) (end 199.971522 82.06) (width 0.2) (layer "F.Cu") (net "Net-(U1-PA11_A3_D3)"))
 (segment (start 141.5 76.5) (end 141.5 62.375) (width 0.2) (layer "F.Cu") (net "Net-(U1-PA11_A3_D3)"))
 (segment (start 199.971522 82.06) (end 200.25 82.06) (width 0.2) (layer "F.Cu") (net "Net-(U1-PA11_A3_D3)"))
 (segment (start 197.9 92.1) (end 157.1 92.1) (width 0.2) (layer "F.Cu") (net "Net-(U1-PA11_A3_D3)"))
 (segment (start 155.69 69.5) (end 159.79 73.6) (width 0.2) (layer "F.Cu") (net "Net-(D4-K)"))
 (segment (start 166.202944 73.6) (end 174.342944 65.46) (width 0.2) (layer "F.Cu") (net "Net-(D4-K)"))
 (segment (start 159.79 73.6) (end 166.202944 73.6) (width 0.2) (layer "F.Cu") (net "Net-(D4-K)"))
 (segment (start 174.342944 65.46) (end 174.77 65.46) (width 0.2) (layer "F.Cu") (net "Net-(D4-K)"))
 (segment (start 181.1 82.1) (end 161.9 82.1) (width 0.2) (layer "B.Cu") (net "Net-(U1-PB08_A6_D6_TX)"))
 (segment (start 161.9 82.1) (end 149.12 69.32) (width 0.2) (layer "B.Cu") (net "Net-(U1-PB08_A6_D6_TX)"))
 (segment (start 149.12 69.32) (end 149.12 62.375) (width 0.2) (layer "B.Cu") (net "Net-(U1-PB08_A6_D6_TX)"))
 (segment (start 152.5 66.69) (end 152.5 81.59) (width 0.2) (layer "F.Cu") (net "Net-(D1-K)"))
 (segment (start 152.5 81.59) (end 155.55 84.64) (width 0.2) (layer "F.Cu") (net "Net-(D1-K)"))
 (segment (start 155.69 63.5) (end 152.5 66.69) (width 0.2) (layer "F.Cu") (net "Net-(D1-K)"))
 (segment (start 149.625 47.125) (end 165 62.5) (width 0.2) (layer "F.Cu") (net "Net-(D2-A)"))
 (segment (start 165 67.81) (end 163.31 69.5) (width 0.2) (layer "F.Cu") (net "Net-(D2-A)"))
 (segment (start 163.31 69.5) (end 163.31 72.5) (width 0.2) (layer "F.Cu") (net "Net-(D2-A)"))
 (segment (start 149.12 47.125) (end 149.625 47.125) (width 0.2) (layer "F.Cu") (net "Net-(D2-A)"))
 (segment (start 165 62.5) (end 165 67.81) (width 0.2) (layer "F.Cu") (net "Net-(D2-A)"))
 (segment (start 154 66.5) (end 153.5 67) (width 0.2) (layer "F.Cu") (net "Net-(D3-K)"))
 (segment (start 193.472944 84.6) (end 193.9 84.6) (width 0.2) (layer "F.Cu") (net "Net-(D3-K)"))
 (segment (start 187.072944 91) (end 193.472944 84.6) (width 0.2) (layer "F.Cu") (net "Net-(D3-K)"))
 (segment (start 155.69 66.5) (end 154 66.5) (width 0.2) (layer "F.Cu") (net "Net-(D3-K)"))
 (segment (start 153.5 77.937056) (end 166.562944 91) (width 0.2) (layer "F.Cu") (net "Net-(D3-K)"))
 (segment (start 153.5 67) (end 153.5 77.937056) (width 0.2) (layer "F.Cu") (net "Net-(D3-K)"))
 (segment (start 166.562944 91) (end 187.072944 91) (width 0.2) (layer "F.Cu") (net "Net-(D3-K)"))
 (segment (start 163.31 63.5) (end 163.31 66.5) (width 0.2) (layer "F.Cu") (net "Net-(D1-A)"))
 (segment (start 146.58 47.125) (end 146.935 47.125) (width 0.2) (layer "F.Cu") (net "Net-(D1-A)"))
 (segment (start 146.935 47.125) (end 163.31 63.5) (width 0.2) (layer "F.Cu") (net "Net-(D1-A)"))
 (segment (start 155.69 72.5) (end 167.83 84.64) (width 0.2) (layer "F.Cu") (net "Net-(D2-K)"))
 (segment (start 167.83 84.64) (end 174.75 84.64) (width 0.2) (layer "F.Cu") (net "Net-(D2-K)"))
 (segment (start 190.25 68) (end 192.75 65.5) (width 0.2) (layer "B.Cu") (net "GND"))
 (segment (start 161.5 53.62) (end 175.87 53.62) (width 0.2) (layer "B.Cu") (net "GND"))
 (segment (start 142.915 53.62) (end 136.42 47.125) (width 0.2) (layer "B.Cu") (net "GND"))
 (segment (start 192.75 65.5) (end 204.75 65.5) (width 0.2) (layer "B.Cu") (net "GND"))
 (segment (start 175.87 53.62) (end 190.25 68) (width 0.2) (layer "B.Cu") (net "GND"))
 (segment (start 161.5 53.62) (end 142.915 53.62) (width 0.2) (layer "B.Cu") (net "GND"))
 (segment (start 140.5 42.5) (end 138.96 44.04) (width 0.2) (layer "F.Cu") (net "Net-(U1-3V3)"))
 (segment (start 138.96 44.04) (end 138.96 47.125) (width 0.2) (layer "F.Cu") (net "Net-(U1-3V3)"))
 (segment (start 161.025 42.5) (end 140.5 42.5) (width 0.2) (layer "F.Cu") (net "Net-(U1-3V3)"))
 (segment (start 163.5 44.975) (end 161.025 42.5) (width 0.2) (layer "F.Cu") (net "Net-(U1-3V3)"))
 (segment (start 161.5 51.08) (end 163.5 49.08) (width 0.2) (layer "F.Cu") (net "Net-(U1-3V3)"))
 (segment (start 163.5 49.08) (end 163.5 44.975) (width 0.2) (layer "F.Cu") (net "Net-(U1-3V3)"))
 (segment (start 157 44) (end 146.128654 44) (width 0.2) (layer "F.Cu") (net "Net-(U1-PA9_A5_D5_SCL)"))
 (segment (start 161.5 48.5) (end 157 44) (width 0.2) (layer "F.Cu") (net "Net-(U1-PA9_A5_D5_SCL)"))
 (segment (start 146.128654 44) (end 145.43 44.698654) (width 0.2) (layer "F.Cu") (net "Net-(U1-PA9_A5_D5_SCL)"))
 (segment (start 145.43 44.698654) (end 145.43 61.225) (width 0.2) (layer "F.Cu") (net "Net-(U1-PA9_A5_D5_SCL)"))
 (segment (start 145.43 61.225) (end 146.58 62.375) (width 0.2) (layer "F.Cu") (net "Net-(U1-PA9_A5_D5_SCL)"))
 (segment (start 161.5 48.54) (end 161.5 48.5) (width 0.2) (layer "F.Cu") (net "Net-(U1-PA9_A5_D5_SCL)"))
 (segment (start 159 43.5) (end 161.5 46) (width 0.2) (layer "F.Cu") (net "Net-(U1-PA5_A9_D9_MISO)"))
 (segment (start 144.04 44.46) (end 145 43.5) (width 0.2) (layer "F.Cu") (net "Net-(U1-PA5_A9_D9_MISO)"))
 (segment (start 144.04 47.125) (end 144.04 44.46) (width 0.2) (layer "F.Cu") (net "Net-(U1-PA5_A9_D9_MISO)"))
 (segment (start 145 43.5) (end 159 43.5) (width 0.2) (layer "F.Cu") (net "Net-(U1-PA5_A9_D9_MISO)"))
 (segment (start 135.27 60.985) (end 135.27 43.23) (width 0.2) (layer "B.Cu") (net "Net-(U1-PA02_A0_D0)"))
 (segment (start 135.27 43.23) (end 136 42.5) (width 0.2) (layer "B.Cu") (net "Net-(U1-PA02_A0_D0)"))
 (segment (start 136 42.5) (end 167.25 42.5) (width 0.2) (layer "B.Cu") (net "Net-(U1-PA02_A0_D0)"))
 (segment (start 133.88 62.375) (end 135.27 60.985) (width 0.2) (layer "B.Cu") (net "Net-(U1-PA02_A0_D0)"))
 (segment (start 167.25 42.5) (end 190.25 65.5) (width 0.2) (layer "B.Cu") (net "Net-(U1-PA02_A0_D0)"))
 (segment (start 174.302944 70.5) (end 190.25 70.5) (width 0.2) (layer "B.Cu") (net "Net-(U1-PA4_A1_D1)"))
 (segment (start 137.52 61.275) (end 165.077944 61.275) (width 0.2) (layer "B.Cu") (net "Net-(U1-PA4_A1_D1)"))
 (segment (start 165.077944 61.275) (end 174.302944 70.5) (width 0.2) (layer "B.Cu") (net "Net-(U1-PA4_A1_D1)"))
 (segment (start 136.42 62.375) (end 137.52 61.275) (width 0.2) (layer "B.Cu") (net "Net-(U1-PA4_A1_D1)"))
 (segment (start 204.75 70.5) (end 204.75 87.75) (width 0.2) (layer "F.Cu") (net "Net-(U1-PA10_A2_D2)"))
 (segment (start 138.96 81.96) (end 138.96 62.375) (width 0.2) (layer "F.Cu") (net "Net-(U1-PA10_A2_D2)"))
 (segment (start 150.5 93.5) (end 138.96 81.96) (width 0.2) (layer "F.Cu") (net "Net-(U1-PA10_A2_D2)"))
 (segment (start 199 93.5) (end 150.5 93.5) (width 0.2) (layer "F.Cu") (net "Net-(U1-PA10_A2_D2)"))
 (segment (start 204.75 87.75) (end 199 93.5) (width 0.2) (layer "F.Cu") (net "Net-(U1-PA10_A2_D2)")))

